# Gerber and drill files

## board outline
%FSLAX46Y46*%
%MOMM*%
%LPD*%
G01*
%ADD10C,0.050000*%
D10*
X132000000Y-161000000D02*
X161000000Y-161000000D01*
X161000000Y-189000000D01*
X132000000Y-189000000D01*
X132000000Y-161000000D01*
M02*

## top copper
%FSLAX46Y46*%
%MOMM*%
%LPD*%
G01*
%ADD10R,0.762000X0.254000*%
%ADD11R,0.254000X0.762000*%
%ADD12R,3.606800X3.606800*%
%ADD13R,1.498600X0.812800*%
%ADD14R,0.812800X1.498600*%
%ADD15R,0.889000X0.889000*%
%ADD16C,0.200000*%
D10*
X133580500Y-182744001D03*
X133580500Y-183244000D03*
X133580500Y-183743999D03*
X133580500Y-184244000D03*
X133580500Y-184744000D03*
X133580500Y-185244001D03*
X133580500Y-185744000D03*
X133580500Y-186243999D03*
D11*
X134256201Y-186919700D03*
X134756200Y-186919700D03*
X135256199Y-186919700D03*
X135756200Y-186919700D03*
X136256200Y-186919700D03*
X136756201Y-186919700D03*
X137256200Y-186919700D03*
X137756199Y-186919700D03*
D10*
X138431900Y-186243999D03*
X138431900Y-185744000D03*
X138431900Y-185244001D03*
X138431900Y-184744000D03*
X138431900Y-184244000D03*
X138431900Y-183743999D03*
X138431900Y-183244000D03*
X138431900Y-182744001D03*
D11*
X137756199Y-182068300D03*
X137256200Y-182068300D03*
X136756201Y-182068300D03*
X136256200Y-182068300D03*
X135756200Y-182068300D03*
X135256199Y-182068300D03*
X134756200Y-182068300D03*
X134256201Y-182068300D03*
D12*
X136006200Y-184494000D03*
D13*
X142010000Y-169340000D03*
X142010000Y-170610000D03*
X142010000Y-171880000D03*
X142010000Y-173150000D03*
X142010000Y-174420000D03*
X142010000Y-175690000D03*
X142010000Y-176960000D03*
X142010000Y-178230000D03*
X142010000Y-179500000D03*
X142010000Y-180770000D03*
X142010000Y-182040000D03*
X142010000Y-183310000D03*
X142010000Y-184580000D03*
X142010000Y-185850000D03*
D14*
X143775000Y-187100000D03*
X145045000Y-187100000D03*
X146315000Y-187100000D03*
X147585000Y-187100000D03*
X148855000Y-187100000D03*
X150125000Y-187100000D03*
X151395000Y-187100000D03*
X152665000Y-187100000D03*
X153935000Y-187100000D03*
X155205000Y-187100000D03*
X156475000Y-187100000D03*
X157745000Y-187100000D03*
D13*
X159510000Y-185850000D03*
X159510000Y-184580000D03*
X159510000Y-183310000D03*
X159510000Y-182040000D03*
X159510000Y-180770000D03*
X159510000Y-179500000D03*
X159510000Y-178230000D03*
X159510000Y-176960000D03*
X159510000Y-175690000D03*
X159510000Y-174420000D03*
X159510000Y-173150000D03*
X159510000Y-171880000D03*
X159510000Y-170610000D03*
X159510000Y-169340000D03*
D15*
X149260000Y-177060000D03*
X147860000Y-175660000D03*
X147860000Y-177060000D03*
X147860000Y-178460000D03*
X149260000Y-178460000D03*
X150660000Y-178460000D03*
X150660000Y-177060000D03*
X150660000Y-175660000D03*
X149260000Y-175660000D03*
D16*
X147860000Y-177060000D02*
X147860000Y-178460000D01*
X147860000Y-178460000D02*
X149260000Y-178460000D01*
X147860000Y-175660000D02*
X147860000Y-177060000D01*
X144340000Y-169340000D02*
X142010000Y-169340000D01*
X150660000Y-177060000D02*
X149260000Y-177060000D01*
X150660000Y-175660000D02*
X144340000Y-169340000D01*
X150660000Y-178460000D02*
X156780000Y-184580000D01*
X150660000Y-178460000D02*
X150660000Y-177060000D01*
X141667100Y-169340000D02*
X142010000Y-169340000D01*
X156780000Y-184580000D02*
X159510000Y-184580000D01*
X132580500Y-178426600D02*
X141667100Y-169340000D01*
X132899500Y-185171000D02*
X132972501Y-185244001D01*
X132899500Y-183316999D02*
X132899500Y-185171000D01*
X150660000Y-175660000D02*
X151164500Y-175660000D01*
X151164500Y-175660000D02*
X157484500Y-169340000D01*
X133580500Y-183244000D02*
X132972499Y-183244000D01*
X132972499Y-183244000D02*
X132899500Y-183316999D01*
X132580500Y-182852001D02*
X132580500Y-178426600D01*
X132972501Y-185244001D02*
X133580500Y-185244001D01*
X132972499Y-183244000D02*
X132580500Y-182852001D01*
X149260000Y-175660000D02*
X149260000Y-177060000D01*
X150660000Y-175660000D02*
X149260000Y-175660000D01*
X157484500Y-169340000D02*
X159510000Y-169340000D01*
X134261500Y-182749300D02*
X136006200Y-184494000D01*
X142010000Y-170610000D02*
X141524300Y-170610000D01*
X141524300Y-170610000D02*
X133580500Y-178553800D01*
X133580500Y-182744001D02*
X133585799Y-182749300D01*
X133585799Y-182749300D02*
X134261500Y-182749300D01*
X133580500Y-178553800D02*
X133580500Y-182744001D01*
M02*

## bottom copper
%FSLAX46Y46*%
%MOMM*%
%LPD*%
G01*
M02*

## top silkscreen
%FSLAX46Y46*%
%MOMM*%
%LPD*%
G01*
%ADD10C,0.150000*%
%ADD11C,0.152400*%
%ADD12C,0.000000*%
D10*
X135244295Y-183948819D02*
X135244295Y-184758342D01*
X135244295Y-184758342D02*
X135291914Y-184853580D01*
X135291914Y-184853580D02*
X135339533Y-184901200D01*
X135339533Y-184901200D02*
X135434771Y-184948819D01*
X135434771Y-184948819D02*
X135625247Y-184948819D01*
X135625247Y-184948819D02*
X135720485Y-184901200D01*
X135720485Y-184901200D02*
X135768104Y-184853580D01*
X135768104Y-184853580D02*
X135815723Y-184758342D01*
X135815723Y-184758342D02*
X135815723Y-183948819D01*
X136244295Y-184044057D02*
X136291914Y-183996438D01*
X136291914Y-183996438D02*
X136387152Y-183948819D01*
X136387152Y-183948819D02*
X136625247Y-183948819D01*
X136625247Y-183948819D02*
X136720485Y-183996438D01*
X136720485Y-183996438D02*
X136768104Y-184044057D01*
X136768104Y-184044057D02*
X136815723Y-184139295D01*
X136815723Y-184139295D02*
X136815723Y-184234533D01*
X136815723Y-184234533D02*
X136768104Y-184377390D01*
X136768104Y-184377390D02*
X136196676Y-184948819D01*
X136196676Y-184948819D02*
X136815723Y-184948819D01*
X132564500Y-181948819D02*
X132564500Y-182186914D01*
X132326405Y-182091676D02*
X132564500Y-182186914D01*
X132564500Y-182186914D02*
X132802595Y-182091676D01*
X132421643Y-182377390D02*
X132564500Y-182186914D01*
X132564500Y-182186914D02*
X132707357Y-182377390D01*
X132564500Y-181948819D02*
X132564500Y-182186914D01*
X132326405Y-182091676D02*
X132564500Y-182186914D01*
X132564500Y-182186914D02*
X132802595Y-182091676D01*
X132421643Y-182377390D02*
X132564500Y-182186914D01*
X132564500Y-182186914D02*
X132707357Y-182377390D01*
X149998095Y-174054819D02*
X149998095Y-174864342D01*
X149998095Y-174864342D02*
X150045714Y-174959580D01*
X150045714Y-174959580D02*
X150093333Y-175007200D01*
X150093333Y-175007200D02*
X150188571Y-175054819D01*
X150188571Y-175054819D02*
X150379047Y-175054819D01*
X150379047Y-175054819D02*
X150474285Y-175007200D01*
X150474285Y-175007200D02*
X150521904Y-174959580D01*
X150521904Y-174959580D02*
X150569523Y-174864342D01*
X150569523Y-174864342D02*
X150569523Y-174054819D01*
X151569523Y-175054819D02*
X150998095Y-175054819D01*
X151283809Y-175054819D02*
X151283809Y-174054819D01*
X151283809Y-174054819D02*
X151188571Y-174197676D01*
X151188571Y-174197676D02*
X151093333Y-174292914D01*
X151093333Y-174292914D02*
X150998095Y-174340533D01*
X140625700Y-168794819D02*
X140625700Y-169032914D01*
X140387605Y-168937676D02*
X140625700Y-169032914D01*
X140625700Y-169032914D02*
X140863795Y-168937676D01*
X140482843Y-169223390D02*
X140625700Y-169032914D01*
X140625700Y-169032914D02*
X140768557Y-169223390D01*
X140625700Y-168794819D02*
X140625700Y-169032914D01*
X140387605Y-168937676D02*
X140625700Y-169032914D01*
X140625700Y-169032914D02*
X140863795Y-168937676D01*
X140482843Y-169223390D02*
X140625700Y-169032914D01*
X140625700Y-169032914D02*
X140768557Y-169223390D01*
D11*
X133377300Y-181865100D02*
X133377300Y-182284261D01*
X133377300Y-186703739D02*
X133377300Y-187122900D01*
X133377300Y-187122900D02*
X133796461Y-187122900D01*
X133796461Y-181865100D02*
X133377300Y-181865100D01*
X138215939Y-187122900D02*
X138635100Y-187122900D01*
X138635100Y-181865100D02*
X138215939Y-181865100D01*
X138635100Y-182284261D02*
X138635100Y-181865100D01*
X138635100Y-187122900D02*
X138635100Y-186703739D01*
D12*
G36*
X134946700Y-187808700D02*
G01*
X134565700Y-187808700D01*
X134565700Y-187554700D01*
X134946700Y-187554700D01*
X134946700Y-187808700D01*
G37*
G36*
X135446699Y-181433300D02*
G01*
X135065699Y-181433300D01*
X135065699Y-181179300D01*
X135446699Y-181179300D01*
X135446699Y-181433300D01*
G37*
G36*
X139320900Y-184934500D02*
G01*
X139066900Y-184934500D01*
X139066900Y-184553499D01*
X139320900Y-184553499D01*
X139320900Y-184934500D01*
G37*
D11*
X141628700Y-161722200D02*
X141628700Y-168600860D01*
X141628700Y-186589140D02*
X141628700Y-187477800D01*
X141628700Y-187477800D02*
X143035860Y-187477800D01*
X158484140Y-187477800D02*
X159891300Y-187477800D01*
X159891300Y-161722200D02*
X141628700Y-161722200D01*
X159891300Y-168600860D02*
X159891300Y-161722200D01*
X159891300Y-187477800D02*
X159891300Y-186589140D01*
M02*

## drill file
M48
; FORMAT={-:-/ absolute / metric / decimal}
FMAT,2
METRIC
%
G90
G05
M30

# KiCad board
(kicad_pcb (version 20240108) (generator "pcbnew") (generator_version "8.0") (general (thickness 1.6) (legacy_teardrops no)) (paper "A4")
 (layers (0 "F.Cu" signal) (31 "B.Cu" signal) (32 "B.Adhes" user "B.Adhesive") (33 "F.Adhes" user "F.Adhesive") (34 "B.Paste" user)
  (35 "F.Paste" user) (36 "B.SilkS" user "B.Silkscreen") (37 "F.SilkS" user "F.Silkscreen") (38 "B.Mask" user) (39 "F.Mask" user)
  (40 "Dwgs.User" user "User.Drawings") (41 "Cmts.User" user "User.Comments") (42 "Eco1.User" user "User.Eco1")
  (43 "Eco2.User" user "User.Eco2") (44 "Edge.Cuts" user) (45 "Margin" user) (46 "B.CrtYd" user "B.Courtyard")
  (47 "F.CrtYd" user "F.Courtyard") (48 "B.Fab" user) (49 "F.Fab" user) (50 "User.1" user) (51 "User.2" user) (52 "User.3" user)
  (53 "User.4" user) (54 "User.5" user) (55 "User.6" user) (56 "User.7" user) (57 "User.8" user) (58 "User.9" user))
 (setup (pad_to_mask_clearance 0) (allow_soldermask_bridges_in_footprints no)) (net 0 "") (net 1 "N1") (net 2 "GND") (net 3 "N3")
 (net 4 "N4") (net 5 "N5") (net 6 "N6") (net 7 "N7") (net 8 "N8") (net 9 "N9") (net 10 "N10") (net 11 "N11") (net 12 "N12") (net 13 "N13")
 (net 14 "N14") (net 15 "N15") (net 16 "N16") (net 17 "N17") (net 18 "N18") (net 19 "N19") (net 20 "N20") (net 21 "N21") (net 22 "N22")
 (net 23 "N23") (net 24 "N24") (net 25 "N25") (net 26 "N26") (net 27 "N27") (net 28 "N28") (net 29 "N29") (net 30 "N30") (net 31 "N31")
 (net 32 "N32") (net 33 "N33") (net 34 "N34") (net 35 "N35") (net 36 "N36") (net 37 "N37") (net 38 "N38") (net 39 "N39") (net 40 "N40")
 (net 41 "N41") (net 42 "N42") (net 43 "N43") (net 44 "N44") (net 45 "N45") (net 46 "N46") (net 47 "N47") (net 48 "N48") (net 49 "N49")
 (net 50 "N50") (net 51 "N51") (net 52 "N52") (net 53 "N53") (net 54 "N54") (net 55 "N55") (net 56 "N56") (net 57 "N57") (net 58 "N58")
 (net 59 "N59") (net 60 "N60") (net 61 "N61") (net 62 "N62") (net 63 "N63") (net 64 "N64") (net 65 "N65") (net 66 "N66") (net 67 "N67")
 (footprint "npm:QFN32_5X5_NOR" (layer "F.Cu") (at 136.0062 184.494)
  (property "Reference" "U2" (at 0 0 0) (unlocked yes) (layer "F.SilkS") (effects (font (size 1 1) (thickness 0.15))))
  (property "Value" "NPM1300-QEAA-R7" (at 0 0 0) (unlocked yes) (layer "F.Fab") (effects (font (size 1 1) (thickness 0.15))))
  (fp_line (start -2.6289 -2.6289) (end -2.6289 -2.209739) (stroke (width 0.1524) (type solid)) (layer "F.SilkS"))
  (fp_line (start -2.6289 2.209739) (end -2.6289 2.6289) (stroke (width 0.1524) (type solid)) (layer "F.SilkS"))
  (fp_line (start -2.6289 2.6289) (end -2.209739 2.6289) (stroke (width 0.1524) (type solid)) (layer "F.SilkS"))
  (fp_line (start -2.209739 -2.6289) (end -2.6289 -2.6289) (stroke (width 0.1524) (type solid)) (layer "F.SilkS"))
  (fp_line (start 2.209739 2.6289) (end 2.6289 2.6289) (stroke (width 0.1524) (type solid)) (layer "F.SilkS"))
  (fp_line (start 2.6289 -2.6289) (end 2.209739 -2.6289) (stroke (width 0.1524) (type solid)) (layer "F.SilkS"))
  (fp_line (start 2.6289 -2.209739) (end 2.6289 -2.6289) (stroke (width 0.1524) (type solid)) (layer "F.SilkS"))
  (fp_line (start 2.6289 2.6289) (end 2.6289 2.209739) (stroke (width 0.1524) (type solid)) (layer "F.SilkS"))
  (fp_poly
   (pts (xy -1.4405 3.0607) (xy -1.4405 3.3147) (xy -1.0595 3.3147) (xy -1.0595 3.0607)) (stroke (width 0) (type solid)) (fill solid)
   (layer "F.SilkS"))
  (fp_poly
   (pts (xy -0.940501 -3.0607) (xy -0.940501 -3.3147) (xy -0.559501 -3.3147) (xy -0.559501 -3.0607)) (stroke (width 0) (type solid))
   (fill solid) (layer "F.SilkS"))
  (fp_poly
   (pts (xy 3.3147 0.059499) (xy 3.3147 0.4405) (xy 3.0607 0.4405) (xy 3.0607 0.059499)) (stroke (width 0) (type solid)) (fill solid)
   (layer "F.SilkS"))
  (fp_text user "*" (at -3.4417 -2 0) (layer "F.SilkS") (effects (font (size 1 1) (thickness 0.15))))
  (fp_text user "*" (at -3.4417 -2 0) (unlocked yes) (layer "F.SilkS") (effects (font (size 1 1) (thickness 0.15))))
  (pad "1" smd rect (at -2.4257 -1.749999 90) (size 0.254 0.762) (layers "F.Cu" "F.Paste" "F.Mask") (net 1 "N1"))
  (pad "2" smd rect (at -2.4257 -1.25 90) (size 0.254 0.762) (layers "F.Cu" "F.Paste" "F.Mask") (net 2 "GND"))
  (pad "3" smd rect (at -2.4257 -0.750001 90) (size 0.254 0.762) (layers "F.Cu" "F.Paste" "F.Mask") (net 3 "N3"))
  (pad "4" smd rect (at -2.4257 -0.25 90) (size 0.254 0.762) (layers "F.Cu" "F.Paste" "F.Mask") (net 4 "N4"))
  (pad "5" smd rect (at -2.4257 0.25 90) (size 0.254 0.762) (layers "F.Cu" "F.Paste" "F.Mask") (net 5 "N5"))
  (pad "6" smd rect (at -2.4257 0.750001 90) (size 0.254 0.762) (layers "F.Cu" "F.Paste" "F.Mask") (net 2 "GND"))
  (pad "7" smd rect (at -2.4257 1.25 90) (size 0.254 0.762) (layers "F.Cu" "F.Paste" "F.Mask") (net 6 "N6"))
  (pad "8" smd rect (at -2.4257 1.749999 90) (size 0.254 0.762) (layers "F.Cu" "F.Paste" "F.Mask") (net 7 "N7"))
  (pad "9" smd rect (at -1.749999 2.4257) (size 0.254 0.762) (layers "F.Cu" "F.Paste" "F.Mask") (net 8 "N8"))
  (pad "10" smd rect (at -1.25 2.4257) (size 0.254 0.762) (layers "F.Cu" "F.Paste" "F.Mask") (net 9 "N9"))
  (pad "11" smd rect (at -0.750001 2.4257) (size 0.254 0.762) (layers "F.Cu" "F.Paste" "F.Mask") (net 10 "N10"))
  (pad "12" smd rect (at -0.25 2.4257) (size 0.254 0.762) (layers "F.Cu" "F.Paste" "F.Mask") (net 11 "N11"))
  (pad "13" smd rect (at 0.25 2.4257) (size 0.254 0.762) (layers "F.Cu" "F.Paste" "F.Mask") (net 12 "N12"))
  (pad "14" smd rect (at 0.750001 2.4257) (size 0.254 0.762) (layers "F.Cu" "F.Paste" "F.Mask") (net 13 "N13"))
  (pad "15" smd rect (at 1.25 2.4257) (size 0.254 0.762) (layers "F.Cu" "F.Paste" "F.Mask") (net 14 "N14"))
  (pad "16" smd rect (at 1.749999 2.4257) (size 0.254 0.762) (layers "F.Cu" "F.Paste" "F.Mask") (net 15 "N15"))
  (pad "17" smd rect (at 2.4257 1.749999 90) (size 0.254 0.762) (layers "F.Cu" "F.Paste" "F.Mask") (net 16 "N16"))
  (pad "18" smd rect (at 2.4257 1.25 90) (size 0.254 0.762) (layers "F.Cu" "F.Paste" "F.Mask") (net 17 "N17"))
  (pad "19" smd rect (at 2.4257 0.750001 90) (size 0.254 0.762) (layers "F.Cu" "F.Paste" "F.Mask") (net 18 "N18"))
  (pad "20" smd rect (at 2.4257 0.25 90) (size 0.254 0.762) (layers "F.Cu" "F.Paste" "F.Mask") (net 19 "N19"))
  (pad "21" smd rect (at 2.4257 -0.25 90) (size 0.254 0.762) (layers "F.Cu" "F.Paste" "F.Mask") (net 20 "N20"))
  (pad "22" smd rect (at 2.4257 -0.750001 90) (size 0.254 0.762) (layers "F.Cu" "F.Paste" "F.Mask") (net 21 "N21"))
  (pad "23" smd rect (at 2.4257 -1.25 90) (size 0.254 0.762) (layers "F.Cu" "F.Paste" "F.Mask") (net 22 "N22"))
  (pad "24" smd rect (at 2.4257 -1.749999 90) (size 0.254 0.762) (layers "F.Cu" "F.Paste" "F.Mask") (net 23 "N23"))
  (pad "25" smd rect (at 1.749999 -2.4257) (size 0.254 0.762) (layers "F.Cu" "F.Paste" "F.Mask") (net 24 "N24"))
  (pad "26" smd rect (at 1.25 -2.4257) (size 0.254 0.762) (layers "F.Cu" "F.Paste" "F.Mask") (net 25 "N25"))
  (pad "27" smd rect (at 0.750001 -2.4257) (size 0.254 0.762) (layers "F.Cu" "F.Paste" "F.Mask") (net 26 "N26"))
  (pad "28" smd rect (at 0.25 -2.4257) (size 0.254 0.762) (layers "F.Cu" "F.Paste" "F.Mask") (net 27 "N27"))
  (pad "29" smd rect (at -0.25 -2.4257) (size 0.254 0.762) (layers "F.Cu" "F.Paste" "F.Mask") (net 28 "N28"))
  (pad "30" smd rect (at -0.750001 -2.4257) (size 0.254 0.762) (layers "F.Cu" "F.Paste" "F.Mask") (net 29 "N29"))
  (pad "31" smd rect (at -1.25 -2.4257) (size 0.254 0.762) (layers "F.Cu" "F.Paste" "F.Mask") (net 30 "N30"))
  (pad "32" smd rect (at -1.749999 -2.4257) (size 0.254 0.762) (layers "F.Cu" "F.Paste" "F.Mask") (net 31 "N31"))
  (pad "33" smd rect (at 0 0) (size 3.6068 3.6068) (layers "F.Cu" "F.Paste" "F.Mask") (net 1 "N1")))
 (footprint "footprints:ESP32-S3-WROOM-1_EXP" (layer "F.Cu") (at 150.76 174.6)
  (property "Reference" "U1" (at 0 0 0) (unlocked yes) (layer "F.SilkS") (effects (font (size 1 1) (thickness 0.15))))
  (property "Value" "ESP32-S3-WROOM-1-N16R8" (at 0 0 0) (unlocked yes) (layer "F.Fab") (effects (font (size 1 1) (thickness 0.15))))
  (fp_line (start -9.1313 -12.8778) (end -9.1313 -5.99914) (stroke (width 0.1524) (type solid)) (layer "F.SilkS"))
  (fp_line (start -9.1313 11.98914) (end -9.1313 12.8778) (stroke (width 0.1524) (type solid)) (layer "F.SilkS"))
  (fp_line (start -9.1313 12.8778) (end -7.72414 12.8778) (stroke (width 0.1524) (type solid)) (layer "F.SilkS"))
  (fp_line (start 7.72414 12.8778) (end 9.1313 12.8778) (stroke (width 0.1524) (type solid)) (layer "F.SilkS"))
  (fp_line (start 9.1313 -12.8778) (end -9.1313 -12.8778) (stroke (width 0.1524) (type solid)) (layer "F.SilkS"))
  (fp_line (start 9.1313 -5.99914) (end 9.1313 -12.8778) (stroke (width 0.1524) (type solid)) (layer "F.SilkS"))
  (fp_line (start 9.1313 12.8778) (end 9.1313 11.98914) (stroke (width 0.1524) (type solid)) (layer "F.SilkS"))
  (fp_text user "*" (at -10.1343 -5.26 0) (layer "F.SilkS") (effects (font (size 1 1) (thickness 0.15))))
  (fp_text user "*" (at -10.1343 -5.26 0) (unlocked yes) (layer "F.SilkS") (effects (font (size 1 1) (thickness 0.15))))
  (pad "1" smd rect (at -8.75 -5.26) (size 1.4986 0.8128) (layers "F.Cu" "F.Paste" "F.Mask") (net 2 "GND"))
  (pad "2" smd rect (at -8.75 -3.99) (size 1.4986 0.8128) (layers "F.Cu" "F.Paste" "F.Mask") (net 1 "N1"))
  (pad "3" smd rect (at -8.75 -2.72) (size 1.4986 0.8128) (layers "F.Cu" "F.Paste" "F.Mask") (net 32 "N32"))
  (pad "4" smd rect (at -8.75 -1.45) (size 1.4986 0.8128) (layers "F.Cu" "F.Paste" "F.Mask") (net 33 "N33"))
  (pad "5" smd rect (at -8.75 -0.18) (size 1.4986 0.8128) (layers "F.Cu" "F.Paste" "F.Mask") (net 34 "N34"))
  (pad "6" smd rect (at -8.75 1.09) (size 1.4986 0.8128) (layers "F.Cu" "F.Paste" "F.Mask") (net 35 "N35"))
  (pad "7" smd rect (at -8.75 2.36) (size 1.4986 0.8128) (layers "F.Cu" "F.Paste" "F.Mask") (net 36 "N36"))
  (pad "8" smd rect (at -8.75 3.63) (size 1.4986 0.8128) (layers "F.Cu" "F.Paste" "F.Mask") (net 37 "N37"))
  (pad "9" smd rect (at -8.75 4.9) (size 1.4986 0.8128) (layers "F.Cu" "F.Paste" "F.Mask") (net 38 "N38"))
  (pad "10" smd rect (at -8.75 6.17) (size 1.4986 0.8128) (layers "F.Cu" "F.Paste" "F.Mask") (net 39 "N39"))
  (pad "11" smd rect (at -8.75 7.44) (size 1.4986 0.8128) (layers "F.Cu" "F.Paste" "F.Mask") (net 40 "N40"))
  (pad "12" smd rect (at -8.75 8.71) (size 1.4986 0.8128) (layers "F.Cu" "F.Paste" "F.Mask") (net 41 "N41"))
  (pad "13" smd rect (at -8.75 9.98) (size 1.4986 0.8128) (layers "F.Cu" "F.Paste" "F.Mask") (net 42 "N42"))
  (pad "14" smd rect (at -8.75 11.25) (size 1.4986 0.8128) (layers "F.Cu" "F.Paste" "F.Mask") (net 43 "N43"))
  (pad "15" smd rect (at -6.985 12.5 90) (size 1.4986 0.8128) (layers "F.Cu" "F.Paste" "F.Mask") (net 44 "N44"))
  (pad "16" smd rect (at -5.715 12.5 90) (size 1.4986 0.8128) (layers "F.Cu" "F.Paste" "F.Mask") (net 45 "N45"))
  (pad "17" smd rect (at -4.445 12.5 90) (size 1.4986 0.8128) (layers "F.Cu" "F.Paste" "F.Mask") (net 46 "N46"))
  (pad "18" smd rect (at -3.175 12.5 90) (size 1.4986 0.8128) (layers "F.Cu" "F.Paste" "F.Mask") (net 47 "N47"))
  (pad "19" smd rect (at -1.905 12.5 90) (size 1.4986 0.8128) (layers "F.Cu" "F.Paste" "F.Mask") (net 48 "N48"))
  (pad "20" smd rect (at -0.635 12.5 90) (size 1.4986 0.8128) (layers "F.Cu" "F.Paste" "F.Mask") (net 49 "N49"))
  (pad "21" smd rect (at 0.635 12.5 90) (size 1.4986 0.8128) (layers "F.Cu" "F.Paste" "F.Mask") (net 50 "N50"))
  (pad "22" smd rect (at 1.905 12.5 90) (size 1.4986 0.8128) (layers "F.Cu" "F.Paste" "F.Mask") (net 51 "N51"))
  (pad "23" smd rect (at 3.175 12.5 90) (size 1.4986 0.8128) (layers "F.Cu" "F.Paste" "F.Mask") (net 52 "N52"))
  (pad "24" smd rect (at 4.445 12.5 90) (size 1.4986 0.8128) (layers "F.Cu" "F.Paste" "F.Mask") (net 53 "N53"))
  (pad "25" smd rect (at 5.715 12.5 90) (size 1.4986 0.8128) (layers "F.Cu" "F.Paste" "F.Mask") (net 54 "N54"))
  (pad "26" smd rect (at 6.985 12.5 90) (size 1.4986 0.8128) (layers "F.Cu" "F.Paste" "F.Mask") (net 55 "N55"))
  (pad "27" smd rect (at 8.75 11.25) (size 1.4986 0.8128) (layers "F.Cu" "F.Paste" "F.Mask") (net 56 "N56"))
  (pad "28" smd rect (at 8.75 9.98) (size 1.4986 0.8128) (layers "F.Cu" "F.Paste" "F.Mask") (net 2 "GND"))
  (pad "29" smd rect (at 8.75 8.71) (size 1.4986 0.8128) (layers "F.Cu" "F.Paste" "F.Mask") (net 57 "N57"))
  (pad "30" smd rect (at 8.75 7.44) (size 1.4986 0.8128) (layers "F.Cu" "F.Paste" "F.Mask") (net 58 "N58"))
  (pad "31" smd rect (at 8.75 6.17) (size 1.4986 0.8128) (layers "F.Cu" "F.Paste" "F.Mask") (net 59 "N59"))
  (pad "32" smd rect (at 8.75 4.9) (size 1.4986 0.8128) (layers "F.Cu" "F.Paste" "F.Mask") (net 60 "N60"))
  (pad "33" smd rect (at 8.75 3.63) (size 1.4986 0.8128) (layers "F.Cu" "F.Paste" "F.Mask") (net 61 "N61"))
  (pad "34" smd rect (at 8.75 2.36) (size 1.4986 0.8128) (layers "F.Cu" "F.Paste" "F.Mask") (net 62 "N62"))
  (pad "35" smd rect (at 8.75 1.09) (size 1.4986 0.8128) (layers "F.Cu" "F.Paste" "F.Mask") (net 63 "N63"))
  (pad "36" smd rect (at 8.75 -0.18) (size 1.4986 0.8128) (layers "F.Cu" "F.Paste" "F.Mask") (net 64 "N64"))
  (pad "37" smd rect (at 8.75 -1.45) (size 1.4986 0.8128) (layers "F.Cu" "F.Paste" "F.Mask") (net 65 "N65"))
  (pad "38" smd rect (at 8.75 -2.72) (size 1.4986 0.8128) (layers "F.Cu" "F.Paste" "F.Mask") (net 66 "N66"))
  (pad "39" smd rect (at 8.75 -3.99) (size 1.4986 0.8128) (layers "F.Cu" "F.Paste" "F.Mask") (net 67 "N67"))
  (pad "40" smd rect (at 8.75 -5.26) (size 1.4986 0.8128) (layers "F.Cu" "F.Paste" "F.Mask") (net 2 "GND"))
  (pad "41" smd rect (at -1.5 2.46) (size 0.889 0.889) (layers "F.Cu" "F.Paste" "F.Mask") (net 2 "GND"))
  (pad "42" smd rect (at -2.9 1.06) (size 0.889 0.889) (layers "F.Cu" "F.Paste" "F.Mask"))
  (pad "43" smd rect (at -2.9 2.46) (size 0.889 0.889) (layers "F.Cu" "F.Paste" "F.Mask"))
  (pad "44" smd rect (at -2.9 3.86) (size 0.889 0.889) (layers "F.Cu" "F.Paste" "F.Mask"))
  (pad "45" smd rect (at -1.5 3.86) (size 0.889 0.889) (layers "F.Cu" "F.Paste" "F.Mask"))
  (pad "46" smd rect (at -0.1 3.86) (size 0.889 0.889) (layers "F.Cu" "F.Paste" "F.Mask") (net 2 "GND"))
  (pad "47" smd rect (at -0.1 2.46) (size 0.889 0.889) (layers "F.Cu" "F.Paste" "F.Mask") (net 2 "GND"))
  (pad "48" smd rect (at -0.1 1.06) (size 0.889 0.889) (layers "F.Cu" "F.Paste" "F.Mask") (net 2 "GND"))
  (pad "49" smd rect (at -1.5 1.06) (size 0.889 0.889) (layers "F.Cu" "F.Paste" "F.Mask") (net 2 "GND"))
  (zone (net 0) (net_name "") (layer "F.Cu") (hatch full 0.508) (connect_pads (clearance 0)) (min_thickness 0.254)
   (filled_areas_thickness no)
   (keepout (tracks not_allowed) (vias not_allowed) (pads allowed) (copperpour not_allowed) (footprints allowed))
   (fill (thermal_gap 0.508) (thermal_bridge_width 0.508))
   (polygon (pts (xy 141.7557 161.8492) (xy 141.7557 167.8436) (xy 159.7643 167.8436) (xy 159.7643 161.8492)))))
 (gr_rect (start 132 161) (end 161 189) (stroke (width 0.05) (type default)) (fill none) (layer "Edge.Cuts"))
 (segment (start 147.86 177.06) (end 147.86 178.46) (width 0.2) (layer "F.Cu") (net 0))
 (segment (start 147.86 178.46) (end 149.26 178.46) (width 0.2) (layer "F.Cu") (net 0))
 (segment (start 147.86 175.66) (end 147.86 177.06) (width 0.2) (layer "F.Cu") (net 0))
 (segment (start 144.34 169.34) (end 142.01 169.34) (width 0.2) (layer "F.Cu") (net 2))
 (segment (start 150.66 177.06) (end 149.26 177.06) (width 0.2) (layer "F.Cu") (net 2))
 (segment (start 150.66 175.66) (end 144.34 169.34) (width 0.2) (layer "F.Cu") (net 2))
 (segment (start 150.66 178.46) (end 156.78 184.58) (width 0.2) (layer "F.Cu") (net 2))
 (segment (start 150.66 178.46) (end 150.66 177.06) (width 0.2) (layer "F.Cu") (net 2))
 (segment (start 141.6671 169.34) (end 142.01 169.34) (width 0.2) (layer "F.Cu") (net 2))
 (segment (start 156.78 184.58) (end 159.51 184.58) (width 0.2) (layer "F.Cu") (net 2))
 (segment (start 132.5805 178.4266) (end 141.6671 169.34) (width 0.2) (layer "F.Cu") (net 2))
 (segment (start 132.8995 185.171) (end 132.972501 185.244001) (width 0.2) (layer "F.Cu") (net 2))
 (segment (start 132.8995 183.316999) (end 132.8995 185.171) (width 0.2) (layer "F.Cu") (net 2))
 (segment (start 150.66 175.66) (end 151.1645 175.66) (width 0.2) (layer "F.Cu") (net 2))
 (segment (start 151.1645 175.66) (end 157.4845 169.34) (width 0.2) (layer "F.Cu") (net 2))
 (segment (start 133.5805 183.244) (end 132.972499 183.244) (width 0.2) (layer "F.Cu") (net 2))
 (segment (start 132.972499 183.244) (end 132.8995 183.316999) (width 0.2) (layer "F.Cu") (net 2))
 (segment (start 132.5805 182.852001) (end 132.5805 178.4266) (width 0.2) (layer "F.Cu") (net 2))
 (segment (start 132.972501 185.244001) (end 133.5805 185.244001) (width 0.2) (layer "F.Cu") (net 2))
 (segment (start 132.972499 183.244) (end 132.5805 182.852001) (width 0.2) (layer "F.Cu") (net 2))
 (segment (start 149.26 175.66) (end 149.26 177.06) (width 0.2) (layer "F.Cu") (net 2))
 (segment (start 150.66 175.66) (end 149.26 175.66) (width 0.2) (layer "F.Cu") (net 2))
 (segment (start 157.4845 169.34) (end 159.51 169.34) (width 0.2) (layer "F.Cu") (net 2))
 (segment (start 134.2615 182.7493) (end 136.0062 184.494) (width 0.2) (layer "F.Cu") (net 1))
 (segment (start 142.01 170.61) (end 141.5243 170.61) (width 0.2) (layer "F.Cu") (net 1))
 (segment (start 141.5243 170.61) (end 133.5805 178.5538) (width 0.2) (layer "F.Cu") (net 1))
 (segment (start 133.5805 182.744001) (end 133.585799 182.7493) (width 0.2) (layer "F.Cu") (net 1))
 (segment (start 133.585799 182.7493) (end 134.2615 182.7493) (width 0.2) (layer "F.Cu") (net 1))
 (segment (start 133.5805 178.5538) (end 133.5805 182.744001) (width 0.2) (layer "F.Cu") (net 1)))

